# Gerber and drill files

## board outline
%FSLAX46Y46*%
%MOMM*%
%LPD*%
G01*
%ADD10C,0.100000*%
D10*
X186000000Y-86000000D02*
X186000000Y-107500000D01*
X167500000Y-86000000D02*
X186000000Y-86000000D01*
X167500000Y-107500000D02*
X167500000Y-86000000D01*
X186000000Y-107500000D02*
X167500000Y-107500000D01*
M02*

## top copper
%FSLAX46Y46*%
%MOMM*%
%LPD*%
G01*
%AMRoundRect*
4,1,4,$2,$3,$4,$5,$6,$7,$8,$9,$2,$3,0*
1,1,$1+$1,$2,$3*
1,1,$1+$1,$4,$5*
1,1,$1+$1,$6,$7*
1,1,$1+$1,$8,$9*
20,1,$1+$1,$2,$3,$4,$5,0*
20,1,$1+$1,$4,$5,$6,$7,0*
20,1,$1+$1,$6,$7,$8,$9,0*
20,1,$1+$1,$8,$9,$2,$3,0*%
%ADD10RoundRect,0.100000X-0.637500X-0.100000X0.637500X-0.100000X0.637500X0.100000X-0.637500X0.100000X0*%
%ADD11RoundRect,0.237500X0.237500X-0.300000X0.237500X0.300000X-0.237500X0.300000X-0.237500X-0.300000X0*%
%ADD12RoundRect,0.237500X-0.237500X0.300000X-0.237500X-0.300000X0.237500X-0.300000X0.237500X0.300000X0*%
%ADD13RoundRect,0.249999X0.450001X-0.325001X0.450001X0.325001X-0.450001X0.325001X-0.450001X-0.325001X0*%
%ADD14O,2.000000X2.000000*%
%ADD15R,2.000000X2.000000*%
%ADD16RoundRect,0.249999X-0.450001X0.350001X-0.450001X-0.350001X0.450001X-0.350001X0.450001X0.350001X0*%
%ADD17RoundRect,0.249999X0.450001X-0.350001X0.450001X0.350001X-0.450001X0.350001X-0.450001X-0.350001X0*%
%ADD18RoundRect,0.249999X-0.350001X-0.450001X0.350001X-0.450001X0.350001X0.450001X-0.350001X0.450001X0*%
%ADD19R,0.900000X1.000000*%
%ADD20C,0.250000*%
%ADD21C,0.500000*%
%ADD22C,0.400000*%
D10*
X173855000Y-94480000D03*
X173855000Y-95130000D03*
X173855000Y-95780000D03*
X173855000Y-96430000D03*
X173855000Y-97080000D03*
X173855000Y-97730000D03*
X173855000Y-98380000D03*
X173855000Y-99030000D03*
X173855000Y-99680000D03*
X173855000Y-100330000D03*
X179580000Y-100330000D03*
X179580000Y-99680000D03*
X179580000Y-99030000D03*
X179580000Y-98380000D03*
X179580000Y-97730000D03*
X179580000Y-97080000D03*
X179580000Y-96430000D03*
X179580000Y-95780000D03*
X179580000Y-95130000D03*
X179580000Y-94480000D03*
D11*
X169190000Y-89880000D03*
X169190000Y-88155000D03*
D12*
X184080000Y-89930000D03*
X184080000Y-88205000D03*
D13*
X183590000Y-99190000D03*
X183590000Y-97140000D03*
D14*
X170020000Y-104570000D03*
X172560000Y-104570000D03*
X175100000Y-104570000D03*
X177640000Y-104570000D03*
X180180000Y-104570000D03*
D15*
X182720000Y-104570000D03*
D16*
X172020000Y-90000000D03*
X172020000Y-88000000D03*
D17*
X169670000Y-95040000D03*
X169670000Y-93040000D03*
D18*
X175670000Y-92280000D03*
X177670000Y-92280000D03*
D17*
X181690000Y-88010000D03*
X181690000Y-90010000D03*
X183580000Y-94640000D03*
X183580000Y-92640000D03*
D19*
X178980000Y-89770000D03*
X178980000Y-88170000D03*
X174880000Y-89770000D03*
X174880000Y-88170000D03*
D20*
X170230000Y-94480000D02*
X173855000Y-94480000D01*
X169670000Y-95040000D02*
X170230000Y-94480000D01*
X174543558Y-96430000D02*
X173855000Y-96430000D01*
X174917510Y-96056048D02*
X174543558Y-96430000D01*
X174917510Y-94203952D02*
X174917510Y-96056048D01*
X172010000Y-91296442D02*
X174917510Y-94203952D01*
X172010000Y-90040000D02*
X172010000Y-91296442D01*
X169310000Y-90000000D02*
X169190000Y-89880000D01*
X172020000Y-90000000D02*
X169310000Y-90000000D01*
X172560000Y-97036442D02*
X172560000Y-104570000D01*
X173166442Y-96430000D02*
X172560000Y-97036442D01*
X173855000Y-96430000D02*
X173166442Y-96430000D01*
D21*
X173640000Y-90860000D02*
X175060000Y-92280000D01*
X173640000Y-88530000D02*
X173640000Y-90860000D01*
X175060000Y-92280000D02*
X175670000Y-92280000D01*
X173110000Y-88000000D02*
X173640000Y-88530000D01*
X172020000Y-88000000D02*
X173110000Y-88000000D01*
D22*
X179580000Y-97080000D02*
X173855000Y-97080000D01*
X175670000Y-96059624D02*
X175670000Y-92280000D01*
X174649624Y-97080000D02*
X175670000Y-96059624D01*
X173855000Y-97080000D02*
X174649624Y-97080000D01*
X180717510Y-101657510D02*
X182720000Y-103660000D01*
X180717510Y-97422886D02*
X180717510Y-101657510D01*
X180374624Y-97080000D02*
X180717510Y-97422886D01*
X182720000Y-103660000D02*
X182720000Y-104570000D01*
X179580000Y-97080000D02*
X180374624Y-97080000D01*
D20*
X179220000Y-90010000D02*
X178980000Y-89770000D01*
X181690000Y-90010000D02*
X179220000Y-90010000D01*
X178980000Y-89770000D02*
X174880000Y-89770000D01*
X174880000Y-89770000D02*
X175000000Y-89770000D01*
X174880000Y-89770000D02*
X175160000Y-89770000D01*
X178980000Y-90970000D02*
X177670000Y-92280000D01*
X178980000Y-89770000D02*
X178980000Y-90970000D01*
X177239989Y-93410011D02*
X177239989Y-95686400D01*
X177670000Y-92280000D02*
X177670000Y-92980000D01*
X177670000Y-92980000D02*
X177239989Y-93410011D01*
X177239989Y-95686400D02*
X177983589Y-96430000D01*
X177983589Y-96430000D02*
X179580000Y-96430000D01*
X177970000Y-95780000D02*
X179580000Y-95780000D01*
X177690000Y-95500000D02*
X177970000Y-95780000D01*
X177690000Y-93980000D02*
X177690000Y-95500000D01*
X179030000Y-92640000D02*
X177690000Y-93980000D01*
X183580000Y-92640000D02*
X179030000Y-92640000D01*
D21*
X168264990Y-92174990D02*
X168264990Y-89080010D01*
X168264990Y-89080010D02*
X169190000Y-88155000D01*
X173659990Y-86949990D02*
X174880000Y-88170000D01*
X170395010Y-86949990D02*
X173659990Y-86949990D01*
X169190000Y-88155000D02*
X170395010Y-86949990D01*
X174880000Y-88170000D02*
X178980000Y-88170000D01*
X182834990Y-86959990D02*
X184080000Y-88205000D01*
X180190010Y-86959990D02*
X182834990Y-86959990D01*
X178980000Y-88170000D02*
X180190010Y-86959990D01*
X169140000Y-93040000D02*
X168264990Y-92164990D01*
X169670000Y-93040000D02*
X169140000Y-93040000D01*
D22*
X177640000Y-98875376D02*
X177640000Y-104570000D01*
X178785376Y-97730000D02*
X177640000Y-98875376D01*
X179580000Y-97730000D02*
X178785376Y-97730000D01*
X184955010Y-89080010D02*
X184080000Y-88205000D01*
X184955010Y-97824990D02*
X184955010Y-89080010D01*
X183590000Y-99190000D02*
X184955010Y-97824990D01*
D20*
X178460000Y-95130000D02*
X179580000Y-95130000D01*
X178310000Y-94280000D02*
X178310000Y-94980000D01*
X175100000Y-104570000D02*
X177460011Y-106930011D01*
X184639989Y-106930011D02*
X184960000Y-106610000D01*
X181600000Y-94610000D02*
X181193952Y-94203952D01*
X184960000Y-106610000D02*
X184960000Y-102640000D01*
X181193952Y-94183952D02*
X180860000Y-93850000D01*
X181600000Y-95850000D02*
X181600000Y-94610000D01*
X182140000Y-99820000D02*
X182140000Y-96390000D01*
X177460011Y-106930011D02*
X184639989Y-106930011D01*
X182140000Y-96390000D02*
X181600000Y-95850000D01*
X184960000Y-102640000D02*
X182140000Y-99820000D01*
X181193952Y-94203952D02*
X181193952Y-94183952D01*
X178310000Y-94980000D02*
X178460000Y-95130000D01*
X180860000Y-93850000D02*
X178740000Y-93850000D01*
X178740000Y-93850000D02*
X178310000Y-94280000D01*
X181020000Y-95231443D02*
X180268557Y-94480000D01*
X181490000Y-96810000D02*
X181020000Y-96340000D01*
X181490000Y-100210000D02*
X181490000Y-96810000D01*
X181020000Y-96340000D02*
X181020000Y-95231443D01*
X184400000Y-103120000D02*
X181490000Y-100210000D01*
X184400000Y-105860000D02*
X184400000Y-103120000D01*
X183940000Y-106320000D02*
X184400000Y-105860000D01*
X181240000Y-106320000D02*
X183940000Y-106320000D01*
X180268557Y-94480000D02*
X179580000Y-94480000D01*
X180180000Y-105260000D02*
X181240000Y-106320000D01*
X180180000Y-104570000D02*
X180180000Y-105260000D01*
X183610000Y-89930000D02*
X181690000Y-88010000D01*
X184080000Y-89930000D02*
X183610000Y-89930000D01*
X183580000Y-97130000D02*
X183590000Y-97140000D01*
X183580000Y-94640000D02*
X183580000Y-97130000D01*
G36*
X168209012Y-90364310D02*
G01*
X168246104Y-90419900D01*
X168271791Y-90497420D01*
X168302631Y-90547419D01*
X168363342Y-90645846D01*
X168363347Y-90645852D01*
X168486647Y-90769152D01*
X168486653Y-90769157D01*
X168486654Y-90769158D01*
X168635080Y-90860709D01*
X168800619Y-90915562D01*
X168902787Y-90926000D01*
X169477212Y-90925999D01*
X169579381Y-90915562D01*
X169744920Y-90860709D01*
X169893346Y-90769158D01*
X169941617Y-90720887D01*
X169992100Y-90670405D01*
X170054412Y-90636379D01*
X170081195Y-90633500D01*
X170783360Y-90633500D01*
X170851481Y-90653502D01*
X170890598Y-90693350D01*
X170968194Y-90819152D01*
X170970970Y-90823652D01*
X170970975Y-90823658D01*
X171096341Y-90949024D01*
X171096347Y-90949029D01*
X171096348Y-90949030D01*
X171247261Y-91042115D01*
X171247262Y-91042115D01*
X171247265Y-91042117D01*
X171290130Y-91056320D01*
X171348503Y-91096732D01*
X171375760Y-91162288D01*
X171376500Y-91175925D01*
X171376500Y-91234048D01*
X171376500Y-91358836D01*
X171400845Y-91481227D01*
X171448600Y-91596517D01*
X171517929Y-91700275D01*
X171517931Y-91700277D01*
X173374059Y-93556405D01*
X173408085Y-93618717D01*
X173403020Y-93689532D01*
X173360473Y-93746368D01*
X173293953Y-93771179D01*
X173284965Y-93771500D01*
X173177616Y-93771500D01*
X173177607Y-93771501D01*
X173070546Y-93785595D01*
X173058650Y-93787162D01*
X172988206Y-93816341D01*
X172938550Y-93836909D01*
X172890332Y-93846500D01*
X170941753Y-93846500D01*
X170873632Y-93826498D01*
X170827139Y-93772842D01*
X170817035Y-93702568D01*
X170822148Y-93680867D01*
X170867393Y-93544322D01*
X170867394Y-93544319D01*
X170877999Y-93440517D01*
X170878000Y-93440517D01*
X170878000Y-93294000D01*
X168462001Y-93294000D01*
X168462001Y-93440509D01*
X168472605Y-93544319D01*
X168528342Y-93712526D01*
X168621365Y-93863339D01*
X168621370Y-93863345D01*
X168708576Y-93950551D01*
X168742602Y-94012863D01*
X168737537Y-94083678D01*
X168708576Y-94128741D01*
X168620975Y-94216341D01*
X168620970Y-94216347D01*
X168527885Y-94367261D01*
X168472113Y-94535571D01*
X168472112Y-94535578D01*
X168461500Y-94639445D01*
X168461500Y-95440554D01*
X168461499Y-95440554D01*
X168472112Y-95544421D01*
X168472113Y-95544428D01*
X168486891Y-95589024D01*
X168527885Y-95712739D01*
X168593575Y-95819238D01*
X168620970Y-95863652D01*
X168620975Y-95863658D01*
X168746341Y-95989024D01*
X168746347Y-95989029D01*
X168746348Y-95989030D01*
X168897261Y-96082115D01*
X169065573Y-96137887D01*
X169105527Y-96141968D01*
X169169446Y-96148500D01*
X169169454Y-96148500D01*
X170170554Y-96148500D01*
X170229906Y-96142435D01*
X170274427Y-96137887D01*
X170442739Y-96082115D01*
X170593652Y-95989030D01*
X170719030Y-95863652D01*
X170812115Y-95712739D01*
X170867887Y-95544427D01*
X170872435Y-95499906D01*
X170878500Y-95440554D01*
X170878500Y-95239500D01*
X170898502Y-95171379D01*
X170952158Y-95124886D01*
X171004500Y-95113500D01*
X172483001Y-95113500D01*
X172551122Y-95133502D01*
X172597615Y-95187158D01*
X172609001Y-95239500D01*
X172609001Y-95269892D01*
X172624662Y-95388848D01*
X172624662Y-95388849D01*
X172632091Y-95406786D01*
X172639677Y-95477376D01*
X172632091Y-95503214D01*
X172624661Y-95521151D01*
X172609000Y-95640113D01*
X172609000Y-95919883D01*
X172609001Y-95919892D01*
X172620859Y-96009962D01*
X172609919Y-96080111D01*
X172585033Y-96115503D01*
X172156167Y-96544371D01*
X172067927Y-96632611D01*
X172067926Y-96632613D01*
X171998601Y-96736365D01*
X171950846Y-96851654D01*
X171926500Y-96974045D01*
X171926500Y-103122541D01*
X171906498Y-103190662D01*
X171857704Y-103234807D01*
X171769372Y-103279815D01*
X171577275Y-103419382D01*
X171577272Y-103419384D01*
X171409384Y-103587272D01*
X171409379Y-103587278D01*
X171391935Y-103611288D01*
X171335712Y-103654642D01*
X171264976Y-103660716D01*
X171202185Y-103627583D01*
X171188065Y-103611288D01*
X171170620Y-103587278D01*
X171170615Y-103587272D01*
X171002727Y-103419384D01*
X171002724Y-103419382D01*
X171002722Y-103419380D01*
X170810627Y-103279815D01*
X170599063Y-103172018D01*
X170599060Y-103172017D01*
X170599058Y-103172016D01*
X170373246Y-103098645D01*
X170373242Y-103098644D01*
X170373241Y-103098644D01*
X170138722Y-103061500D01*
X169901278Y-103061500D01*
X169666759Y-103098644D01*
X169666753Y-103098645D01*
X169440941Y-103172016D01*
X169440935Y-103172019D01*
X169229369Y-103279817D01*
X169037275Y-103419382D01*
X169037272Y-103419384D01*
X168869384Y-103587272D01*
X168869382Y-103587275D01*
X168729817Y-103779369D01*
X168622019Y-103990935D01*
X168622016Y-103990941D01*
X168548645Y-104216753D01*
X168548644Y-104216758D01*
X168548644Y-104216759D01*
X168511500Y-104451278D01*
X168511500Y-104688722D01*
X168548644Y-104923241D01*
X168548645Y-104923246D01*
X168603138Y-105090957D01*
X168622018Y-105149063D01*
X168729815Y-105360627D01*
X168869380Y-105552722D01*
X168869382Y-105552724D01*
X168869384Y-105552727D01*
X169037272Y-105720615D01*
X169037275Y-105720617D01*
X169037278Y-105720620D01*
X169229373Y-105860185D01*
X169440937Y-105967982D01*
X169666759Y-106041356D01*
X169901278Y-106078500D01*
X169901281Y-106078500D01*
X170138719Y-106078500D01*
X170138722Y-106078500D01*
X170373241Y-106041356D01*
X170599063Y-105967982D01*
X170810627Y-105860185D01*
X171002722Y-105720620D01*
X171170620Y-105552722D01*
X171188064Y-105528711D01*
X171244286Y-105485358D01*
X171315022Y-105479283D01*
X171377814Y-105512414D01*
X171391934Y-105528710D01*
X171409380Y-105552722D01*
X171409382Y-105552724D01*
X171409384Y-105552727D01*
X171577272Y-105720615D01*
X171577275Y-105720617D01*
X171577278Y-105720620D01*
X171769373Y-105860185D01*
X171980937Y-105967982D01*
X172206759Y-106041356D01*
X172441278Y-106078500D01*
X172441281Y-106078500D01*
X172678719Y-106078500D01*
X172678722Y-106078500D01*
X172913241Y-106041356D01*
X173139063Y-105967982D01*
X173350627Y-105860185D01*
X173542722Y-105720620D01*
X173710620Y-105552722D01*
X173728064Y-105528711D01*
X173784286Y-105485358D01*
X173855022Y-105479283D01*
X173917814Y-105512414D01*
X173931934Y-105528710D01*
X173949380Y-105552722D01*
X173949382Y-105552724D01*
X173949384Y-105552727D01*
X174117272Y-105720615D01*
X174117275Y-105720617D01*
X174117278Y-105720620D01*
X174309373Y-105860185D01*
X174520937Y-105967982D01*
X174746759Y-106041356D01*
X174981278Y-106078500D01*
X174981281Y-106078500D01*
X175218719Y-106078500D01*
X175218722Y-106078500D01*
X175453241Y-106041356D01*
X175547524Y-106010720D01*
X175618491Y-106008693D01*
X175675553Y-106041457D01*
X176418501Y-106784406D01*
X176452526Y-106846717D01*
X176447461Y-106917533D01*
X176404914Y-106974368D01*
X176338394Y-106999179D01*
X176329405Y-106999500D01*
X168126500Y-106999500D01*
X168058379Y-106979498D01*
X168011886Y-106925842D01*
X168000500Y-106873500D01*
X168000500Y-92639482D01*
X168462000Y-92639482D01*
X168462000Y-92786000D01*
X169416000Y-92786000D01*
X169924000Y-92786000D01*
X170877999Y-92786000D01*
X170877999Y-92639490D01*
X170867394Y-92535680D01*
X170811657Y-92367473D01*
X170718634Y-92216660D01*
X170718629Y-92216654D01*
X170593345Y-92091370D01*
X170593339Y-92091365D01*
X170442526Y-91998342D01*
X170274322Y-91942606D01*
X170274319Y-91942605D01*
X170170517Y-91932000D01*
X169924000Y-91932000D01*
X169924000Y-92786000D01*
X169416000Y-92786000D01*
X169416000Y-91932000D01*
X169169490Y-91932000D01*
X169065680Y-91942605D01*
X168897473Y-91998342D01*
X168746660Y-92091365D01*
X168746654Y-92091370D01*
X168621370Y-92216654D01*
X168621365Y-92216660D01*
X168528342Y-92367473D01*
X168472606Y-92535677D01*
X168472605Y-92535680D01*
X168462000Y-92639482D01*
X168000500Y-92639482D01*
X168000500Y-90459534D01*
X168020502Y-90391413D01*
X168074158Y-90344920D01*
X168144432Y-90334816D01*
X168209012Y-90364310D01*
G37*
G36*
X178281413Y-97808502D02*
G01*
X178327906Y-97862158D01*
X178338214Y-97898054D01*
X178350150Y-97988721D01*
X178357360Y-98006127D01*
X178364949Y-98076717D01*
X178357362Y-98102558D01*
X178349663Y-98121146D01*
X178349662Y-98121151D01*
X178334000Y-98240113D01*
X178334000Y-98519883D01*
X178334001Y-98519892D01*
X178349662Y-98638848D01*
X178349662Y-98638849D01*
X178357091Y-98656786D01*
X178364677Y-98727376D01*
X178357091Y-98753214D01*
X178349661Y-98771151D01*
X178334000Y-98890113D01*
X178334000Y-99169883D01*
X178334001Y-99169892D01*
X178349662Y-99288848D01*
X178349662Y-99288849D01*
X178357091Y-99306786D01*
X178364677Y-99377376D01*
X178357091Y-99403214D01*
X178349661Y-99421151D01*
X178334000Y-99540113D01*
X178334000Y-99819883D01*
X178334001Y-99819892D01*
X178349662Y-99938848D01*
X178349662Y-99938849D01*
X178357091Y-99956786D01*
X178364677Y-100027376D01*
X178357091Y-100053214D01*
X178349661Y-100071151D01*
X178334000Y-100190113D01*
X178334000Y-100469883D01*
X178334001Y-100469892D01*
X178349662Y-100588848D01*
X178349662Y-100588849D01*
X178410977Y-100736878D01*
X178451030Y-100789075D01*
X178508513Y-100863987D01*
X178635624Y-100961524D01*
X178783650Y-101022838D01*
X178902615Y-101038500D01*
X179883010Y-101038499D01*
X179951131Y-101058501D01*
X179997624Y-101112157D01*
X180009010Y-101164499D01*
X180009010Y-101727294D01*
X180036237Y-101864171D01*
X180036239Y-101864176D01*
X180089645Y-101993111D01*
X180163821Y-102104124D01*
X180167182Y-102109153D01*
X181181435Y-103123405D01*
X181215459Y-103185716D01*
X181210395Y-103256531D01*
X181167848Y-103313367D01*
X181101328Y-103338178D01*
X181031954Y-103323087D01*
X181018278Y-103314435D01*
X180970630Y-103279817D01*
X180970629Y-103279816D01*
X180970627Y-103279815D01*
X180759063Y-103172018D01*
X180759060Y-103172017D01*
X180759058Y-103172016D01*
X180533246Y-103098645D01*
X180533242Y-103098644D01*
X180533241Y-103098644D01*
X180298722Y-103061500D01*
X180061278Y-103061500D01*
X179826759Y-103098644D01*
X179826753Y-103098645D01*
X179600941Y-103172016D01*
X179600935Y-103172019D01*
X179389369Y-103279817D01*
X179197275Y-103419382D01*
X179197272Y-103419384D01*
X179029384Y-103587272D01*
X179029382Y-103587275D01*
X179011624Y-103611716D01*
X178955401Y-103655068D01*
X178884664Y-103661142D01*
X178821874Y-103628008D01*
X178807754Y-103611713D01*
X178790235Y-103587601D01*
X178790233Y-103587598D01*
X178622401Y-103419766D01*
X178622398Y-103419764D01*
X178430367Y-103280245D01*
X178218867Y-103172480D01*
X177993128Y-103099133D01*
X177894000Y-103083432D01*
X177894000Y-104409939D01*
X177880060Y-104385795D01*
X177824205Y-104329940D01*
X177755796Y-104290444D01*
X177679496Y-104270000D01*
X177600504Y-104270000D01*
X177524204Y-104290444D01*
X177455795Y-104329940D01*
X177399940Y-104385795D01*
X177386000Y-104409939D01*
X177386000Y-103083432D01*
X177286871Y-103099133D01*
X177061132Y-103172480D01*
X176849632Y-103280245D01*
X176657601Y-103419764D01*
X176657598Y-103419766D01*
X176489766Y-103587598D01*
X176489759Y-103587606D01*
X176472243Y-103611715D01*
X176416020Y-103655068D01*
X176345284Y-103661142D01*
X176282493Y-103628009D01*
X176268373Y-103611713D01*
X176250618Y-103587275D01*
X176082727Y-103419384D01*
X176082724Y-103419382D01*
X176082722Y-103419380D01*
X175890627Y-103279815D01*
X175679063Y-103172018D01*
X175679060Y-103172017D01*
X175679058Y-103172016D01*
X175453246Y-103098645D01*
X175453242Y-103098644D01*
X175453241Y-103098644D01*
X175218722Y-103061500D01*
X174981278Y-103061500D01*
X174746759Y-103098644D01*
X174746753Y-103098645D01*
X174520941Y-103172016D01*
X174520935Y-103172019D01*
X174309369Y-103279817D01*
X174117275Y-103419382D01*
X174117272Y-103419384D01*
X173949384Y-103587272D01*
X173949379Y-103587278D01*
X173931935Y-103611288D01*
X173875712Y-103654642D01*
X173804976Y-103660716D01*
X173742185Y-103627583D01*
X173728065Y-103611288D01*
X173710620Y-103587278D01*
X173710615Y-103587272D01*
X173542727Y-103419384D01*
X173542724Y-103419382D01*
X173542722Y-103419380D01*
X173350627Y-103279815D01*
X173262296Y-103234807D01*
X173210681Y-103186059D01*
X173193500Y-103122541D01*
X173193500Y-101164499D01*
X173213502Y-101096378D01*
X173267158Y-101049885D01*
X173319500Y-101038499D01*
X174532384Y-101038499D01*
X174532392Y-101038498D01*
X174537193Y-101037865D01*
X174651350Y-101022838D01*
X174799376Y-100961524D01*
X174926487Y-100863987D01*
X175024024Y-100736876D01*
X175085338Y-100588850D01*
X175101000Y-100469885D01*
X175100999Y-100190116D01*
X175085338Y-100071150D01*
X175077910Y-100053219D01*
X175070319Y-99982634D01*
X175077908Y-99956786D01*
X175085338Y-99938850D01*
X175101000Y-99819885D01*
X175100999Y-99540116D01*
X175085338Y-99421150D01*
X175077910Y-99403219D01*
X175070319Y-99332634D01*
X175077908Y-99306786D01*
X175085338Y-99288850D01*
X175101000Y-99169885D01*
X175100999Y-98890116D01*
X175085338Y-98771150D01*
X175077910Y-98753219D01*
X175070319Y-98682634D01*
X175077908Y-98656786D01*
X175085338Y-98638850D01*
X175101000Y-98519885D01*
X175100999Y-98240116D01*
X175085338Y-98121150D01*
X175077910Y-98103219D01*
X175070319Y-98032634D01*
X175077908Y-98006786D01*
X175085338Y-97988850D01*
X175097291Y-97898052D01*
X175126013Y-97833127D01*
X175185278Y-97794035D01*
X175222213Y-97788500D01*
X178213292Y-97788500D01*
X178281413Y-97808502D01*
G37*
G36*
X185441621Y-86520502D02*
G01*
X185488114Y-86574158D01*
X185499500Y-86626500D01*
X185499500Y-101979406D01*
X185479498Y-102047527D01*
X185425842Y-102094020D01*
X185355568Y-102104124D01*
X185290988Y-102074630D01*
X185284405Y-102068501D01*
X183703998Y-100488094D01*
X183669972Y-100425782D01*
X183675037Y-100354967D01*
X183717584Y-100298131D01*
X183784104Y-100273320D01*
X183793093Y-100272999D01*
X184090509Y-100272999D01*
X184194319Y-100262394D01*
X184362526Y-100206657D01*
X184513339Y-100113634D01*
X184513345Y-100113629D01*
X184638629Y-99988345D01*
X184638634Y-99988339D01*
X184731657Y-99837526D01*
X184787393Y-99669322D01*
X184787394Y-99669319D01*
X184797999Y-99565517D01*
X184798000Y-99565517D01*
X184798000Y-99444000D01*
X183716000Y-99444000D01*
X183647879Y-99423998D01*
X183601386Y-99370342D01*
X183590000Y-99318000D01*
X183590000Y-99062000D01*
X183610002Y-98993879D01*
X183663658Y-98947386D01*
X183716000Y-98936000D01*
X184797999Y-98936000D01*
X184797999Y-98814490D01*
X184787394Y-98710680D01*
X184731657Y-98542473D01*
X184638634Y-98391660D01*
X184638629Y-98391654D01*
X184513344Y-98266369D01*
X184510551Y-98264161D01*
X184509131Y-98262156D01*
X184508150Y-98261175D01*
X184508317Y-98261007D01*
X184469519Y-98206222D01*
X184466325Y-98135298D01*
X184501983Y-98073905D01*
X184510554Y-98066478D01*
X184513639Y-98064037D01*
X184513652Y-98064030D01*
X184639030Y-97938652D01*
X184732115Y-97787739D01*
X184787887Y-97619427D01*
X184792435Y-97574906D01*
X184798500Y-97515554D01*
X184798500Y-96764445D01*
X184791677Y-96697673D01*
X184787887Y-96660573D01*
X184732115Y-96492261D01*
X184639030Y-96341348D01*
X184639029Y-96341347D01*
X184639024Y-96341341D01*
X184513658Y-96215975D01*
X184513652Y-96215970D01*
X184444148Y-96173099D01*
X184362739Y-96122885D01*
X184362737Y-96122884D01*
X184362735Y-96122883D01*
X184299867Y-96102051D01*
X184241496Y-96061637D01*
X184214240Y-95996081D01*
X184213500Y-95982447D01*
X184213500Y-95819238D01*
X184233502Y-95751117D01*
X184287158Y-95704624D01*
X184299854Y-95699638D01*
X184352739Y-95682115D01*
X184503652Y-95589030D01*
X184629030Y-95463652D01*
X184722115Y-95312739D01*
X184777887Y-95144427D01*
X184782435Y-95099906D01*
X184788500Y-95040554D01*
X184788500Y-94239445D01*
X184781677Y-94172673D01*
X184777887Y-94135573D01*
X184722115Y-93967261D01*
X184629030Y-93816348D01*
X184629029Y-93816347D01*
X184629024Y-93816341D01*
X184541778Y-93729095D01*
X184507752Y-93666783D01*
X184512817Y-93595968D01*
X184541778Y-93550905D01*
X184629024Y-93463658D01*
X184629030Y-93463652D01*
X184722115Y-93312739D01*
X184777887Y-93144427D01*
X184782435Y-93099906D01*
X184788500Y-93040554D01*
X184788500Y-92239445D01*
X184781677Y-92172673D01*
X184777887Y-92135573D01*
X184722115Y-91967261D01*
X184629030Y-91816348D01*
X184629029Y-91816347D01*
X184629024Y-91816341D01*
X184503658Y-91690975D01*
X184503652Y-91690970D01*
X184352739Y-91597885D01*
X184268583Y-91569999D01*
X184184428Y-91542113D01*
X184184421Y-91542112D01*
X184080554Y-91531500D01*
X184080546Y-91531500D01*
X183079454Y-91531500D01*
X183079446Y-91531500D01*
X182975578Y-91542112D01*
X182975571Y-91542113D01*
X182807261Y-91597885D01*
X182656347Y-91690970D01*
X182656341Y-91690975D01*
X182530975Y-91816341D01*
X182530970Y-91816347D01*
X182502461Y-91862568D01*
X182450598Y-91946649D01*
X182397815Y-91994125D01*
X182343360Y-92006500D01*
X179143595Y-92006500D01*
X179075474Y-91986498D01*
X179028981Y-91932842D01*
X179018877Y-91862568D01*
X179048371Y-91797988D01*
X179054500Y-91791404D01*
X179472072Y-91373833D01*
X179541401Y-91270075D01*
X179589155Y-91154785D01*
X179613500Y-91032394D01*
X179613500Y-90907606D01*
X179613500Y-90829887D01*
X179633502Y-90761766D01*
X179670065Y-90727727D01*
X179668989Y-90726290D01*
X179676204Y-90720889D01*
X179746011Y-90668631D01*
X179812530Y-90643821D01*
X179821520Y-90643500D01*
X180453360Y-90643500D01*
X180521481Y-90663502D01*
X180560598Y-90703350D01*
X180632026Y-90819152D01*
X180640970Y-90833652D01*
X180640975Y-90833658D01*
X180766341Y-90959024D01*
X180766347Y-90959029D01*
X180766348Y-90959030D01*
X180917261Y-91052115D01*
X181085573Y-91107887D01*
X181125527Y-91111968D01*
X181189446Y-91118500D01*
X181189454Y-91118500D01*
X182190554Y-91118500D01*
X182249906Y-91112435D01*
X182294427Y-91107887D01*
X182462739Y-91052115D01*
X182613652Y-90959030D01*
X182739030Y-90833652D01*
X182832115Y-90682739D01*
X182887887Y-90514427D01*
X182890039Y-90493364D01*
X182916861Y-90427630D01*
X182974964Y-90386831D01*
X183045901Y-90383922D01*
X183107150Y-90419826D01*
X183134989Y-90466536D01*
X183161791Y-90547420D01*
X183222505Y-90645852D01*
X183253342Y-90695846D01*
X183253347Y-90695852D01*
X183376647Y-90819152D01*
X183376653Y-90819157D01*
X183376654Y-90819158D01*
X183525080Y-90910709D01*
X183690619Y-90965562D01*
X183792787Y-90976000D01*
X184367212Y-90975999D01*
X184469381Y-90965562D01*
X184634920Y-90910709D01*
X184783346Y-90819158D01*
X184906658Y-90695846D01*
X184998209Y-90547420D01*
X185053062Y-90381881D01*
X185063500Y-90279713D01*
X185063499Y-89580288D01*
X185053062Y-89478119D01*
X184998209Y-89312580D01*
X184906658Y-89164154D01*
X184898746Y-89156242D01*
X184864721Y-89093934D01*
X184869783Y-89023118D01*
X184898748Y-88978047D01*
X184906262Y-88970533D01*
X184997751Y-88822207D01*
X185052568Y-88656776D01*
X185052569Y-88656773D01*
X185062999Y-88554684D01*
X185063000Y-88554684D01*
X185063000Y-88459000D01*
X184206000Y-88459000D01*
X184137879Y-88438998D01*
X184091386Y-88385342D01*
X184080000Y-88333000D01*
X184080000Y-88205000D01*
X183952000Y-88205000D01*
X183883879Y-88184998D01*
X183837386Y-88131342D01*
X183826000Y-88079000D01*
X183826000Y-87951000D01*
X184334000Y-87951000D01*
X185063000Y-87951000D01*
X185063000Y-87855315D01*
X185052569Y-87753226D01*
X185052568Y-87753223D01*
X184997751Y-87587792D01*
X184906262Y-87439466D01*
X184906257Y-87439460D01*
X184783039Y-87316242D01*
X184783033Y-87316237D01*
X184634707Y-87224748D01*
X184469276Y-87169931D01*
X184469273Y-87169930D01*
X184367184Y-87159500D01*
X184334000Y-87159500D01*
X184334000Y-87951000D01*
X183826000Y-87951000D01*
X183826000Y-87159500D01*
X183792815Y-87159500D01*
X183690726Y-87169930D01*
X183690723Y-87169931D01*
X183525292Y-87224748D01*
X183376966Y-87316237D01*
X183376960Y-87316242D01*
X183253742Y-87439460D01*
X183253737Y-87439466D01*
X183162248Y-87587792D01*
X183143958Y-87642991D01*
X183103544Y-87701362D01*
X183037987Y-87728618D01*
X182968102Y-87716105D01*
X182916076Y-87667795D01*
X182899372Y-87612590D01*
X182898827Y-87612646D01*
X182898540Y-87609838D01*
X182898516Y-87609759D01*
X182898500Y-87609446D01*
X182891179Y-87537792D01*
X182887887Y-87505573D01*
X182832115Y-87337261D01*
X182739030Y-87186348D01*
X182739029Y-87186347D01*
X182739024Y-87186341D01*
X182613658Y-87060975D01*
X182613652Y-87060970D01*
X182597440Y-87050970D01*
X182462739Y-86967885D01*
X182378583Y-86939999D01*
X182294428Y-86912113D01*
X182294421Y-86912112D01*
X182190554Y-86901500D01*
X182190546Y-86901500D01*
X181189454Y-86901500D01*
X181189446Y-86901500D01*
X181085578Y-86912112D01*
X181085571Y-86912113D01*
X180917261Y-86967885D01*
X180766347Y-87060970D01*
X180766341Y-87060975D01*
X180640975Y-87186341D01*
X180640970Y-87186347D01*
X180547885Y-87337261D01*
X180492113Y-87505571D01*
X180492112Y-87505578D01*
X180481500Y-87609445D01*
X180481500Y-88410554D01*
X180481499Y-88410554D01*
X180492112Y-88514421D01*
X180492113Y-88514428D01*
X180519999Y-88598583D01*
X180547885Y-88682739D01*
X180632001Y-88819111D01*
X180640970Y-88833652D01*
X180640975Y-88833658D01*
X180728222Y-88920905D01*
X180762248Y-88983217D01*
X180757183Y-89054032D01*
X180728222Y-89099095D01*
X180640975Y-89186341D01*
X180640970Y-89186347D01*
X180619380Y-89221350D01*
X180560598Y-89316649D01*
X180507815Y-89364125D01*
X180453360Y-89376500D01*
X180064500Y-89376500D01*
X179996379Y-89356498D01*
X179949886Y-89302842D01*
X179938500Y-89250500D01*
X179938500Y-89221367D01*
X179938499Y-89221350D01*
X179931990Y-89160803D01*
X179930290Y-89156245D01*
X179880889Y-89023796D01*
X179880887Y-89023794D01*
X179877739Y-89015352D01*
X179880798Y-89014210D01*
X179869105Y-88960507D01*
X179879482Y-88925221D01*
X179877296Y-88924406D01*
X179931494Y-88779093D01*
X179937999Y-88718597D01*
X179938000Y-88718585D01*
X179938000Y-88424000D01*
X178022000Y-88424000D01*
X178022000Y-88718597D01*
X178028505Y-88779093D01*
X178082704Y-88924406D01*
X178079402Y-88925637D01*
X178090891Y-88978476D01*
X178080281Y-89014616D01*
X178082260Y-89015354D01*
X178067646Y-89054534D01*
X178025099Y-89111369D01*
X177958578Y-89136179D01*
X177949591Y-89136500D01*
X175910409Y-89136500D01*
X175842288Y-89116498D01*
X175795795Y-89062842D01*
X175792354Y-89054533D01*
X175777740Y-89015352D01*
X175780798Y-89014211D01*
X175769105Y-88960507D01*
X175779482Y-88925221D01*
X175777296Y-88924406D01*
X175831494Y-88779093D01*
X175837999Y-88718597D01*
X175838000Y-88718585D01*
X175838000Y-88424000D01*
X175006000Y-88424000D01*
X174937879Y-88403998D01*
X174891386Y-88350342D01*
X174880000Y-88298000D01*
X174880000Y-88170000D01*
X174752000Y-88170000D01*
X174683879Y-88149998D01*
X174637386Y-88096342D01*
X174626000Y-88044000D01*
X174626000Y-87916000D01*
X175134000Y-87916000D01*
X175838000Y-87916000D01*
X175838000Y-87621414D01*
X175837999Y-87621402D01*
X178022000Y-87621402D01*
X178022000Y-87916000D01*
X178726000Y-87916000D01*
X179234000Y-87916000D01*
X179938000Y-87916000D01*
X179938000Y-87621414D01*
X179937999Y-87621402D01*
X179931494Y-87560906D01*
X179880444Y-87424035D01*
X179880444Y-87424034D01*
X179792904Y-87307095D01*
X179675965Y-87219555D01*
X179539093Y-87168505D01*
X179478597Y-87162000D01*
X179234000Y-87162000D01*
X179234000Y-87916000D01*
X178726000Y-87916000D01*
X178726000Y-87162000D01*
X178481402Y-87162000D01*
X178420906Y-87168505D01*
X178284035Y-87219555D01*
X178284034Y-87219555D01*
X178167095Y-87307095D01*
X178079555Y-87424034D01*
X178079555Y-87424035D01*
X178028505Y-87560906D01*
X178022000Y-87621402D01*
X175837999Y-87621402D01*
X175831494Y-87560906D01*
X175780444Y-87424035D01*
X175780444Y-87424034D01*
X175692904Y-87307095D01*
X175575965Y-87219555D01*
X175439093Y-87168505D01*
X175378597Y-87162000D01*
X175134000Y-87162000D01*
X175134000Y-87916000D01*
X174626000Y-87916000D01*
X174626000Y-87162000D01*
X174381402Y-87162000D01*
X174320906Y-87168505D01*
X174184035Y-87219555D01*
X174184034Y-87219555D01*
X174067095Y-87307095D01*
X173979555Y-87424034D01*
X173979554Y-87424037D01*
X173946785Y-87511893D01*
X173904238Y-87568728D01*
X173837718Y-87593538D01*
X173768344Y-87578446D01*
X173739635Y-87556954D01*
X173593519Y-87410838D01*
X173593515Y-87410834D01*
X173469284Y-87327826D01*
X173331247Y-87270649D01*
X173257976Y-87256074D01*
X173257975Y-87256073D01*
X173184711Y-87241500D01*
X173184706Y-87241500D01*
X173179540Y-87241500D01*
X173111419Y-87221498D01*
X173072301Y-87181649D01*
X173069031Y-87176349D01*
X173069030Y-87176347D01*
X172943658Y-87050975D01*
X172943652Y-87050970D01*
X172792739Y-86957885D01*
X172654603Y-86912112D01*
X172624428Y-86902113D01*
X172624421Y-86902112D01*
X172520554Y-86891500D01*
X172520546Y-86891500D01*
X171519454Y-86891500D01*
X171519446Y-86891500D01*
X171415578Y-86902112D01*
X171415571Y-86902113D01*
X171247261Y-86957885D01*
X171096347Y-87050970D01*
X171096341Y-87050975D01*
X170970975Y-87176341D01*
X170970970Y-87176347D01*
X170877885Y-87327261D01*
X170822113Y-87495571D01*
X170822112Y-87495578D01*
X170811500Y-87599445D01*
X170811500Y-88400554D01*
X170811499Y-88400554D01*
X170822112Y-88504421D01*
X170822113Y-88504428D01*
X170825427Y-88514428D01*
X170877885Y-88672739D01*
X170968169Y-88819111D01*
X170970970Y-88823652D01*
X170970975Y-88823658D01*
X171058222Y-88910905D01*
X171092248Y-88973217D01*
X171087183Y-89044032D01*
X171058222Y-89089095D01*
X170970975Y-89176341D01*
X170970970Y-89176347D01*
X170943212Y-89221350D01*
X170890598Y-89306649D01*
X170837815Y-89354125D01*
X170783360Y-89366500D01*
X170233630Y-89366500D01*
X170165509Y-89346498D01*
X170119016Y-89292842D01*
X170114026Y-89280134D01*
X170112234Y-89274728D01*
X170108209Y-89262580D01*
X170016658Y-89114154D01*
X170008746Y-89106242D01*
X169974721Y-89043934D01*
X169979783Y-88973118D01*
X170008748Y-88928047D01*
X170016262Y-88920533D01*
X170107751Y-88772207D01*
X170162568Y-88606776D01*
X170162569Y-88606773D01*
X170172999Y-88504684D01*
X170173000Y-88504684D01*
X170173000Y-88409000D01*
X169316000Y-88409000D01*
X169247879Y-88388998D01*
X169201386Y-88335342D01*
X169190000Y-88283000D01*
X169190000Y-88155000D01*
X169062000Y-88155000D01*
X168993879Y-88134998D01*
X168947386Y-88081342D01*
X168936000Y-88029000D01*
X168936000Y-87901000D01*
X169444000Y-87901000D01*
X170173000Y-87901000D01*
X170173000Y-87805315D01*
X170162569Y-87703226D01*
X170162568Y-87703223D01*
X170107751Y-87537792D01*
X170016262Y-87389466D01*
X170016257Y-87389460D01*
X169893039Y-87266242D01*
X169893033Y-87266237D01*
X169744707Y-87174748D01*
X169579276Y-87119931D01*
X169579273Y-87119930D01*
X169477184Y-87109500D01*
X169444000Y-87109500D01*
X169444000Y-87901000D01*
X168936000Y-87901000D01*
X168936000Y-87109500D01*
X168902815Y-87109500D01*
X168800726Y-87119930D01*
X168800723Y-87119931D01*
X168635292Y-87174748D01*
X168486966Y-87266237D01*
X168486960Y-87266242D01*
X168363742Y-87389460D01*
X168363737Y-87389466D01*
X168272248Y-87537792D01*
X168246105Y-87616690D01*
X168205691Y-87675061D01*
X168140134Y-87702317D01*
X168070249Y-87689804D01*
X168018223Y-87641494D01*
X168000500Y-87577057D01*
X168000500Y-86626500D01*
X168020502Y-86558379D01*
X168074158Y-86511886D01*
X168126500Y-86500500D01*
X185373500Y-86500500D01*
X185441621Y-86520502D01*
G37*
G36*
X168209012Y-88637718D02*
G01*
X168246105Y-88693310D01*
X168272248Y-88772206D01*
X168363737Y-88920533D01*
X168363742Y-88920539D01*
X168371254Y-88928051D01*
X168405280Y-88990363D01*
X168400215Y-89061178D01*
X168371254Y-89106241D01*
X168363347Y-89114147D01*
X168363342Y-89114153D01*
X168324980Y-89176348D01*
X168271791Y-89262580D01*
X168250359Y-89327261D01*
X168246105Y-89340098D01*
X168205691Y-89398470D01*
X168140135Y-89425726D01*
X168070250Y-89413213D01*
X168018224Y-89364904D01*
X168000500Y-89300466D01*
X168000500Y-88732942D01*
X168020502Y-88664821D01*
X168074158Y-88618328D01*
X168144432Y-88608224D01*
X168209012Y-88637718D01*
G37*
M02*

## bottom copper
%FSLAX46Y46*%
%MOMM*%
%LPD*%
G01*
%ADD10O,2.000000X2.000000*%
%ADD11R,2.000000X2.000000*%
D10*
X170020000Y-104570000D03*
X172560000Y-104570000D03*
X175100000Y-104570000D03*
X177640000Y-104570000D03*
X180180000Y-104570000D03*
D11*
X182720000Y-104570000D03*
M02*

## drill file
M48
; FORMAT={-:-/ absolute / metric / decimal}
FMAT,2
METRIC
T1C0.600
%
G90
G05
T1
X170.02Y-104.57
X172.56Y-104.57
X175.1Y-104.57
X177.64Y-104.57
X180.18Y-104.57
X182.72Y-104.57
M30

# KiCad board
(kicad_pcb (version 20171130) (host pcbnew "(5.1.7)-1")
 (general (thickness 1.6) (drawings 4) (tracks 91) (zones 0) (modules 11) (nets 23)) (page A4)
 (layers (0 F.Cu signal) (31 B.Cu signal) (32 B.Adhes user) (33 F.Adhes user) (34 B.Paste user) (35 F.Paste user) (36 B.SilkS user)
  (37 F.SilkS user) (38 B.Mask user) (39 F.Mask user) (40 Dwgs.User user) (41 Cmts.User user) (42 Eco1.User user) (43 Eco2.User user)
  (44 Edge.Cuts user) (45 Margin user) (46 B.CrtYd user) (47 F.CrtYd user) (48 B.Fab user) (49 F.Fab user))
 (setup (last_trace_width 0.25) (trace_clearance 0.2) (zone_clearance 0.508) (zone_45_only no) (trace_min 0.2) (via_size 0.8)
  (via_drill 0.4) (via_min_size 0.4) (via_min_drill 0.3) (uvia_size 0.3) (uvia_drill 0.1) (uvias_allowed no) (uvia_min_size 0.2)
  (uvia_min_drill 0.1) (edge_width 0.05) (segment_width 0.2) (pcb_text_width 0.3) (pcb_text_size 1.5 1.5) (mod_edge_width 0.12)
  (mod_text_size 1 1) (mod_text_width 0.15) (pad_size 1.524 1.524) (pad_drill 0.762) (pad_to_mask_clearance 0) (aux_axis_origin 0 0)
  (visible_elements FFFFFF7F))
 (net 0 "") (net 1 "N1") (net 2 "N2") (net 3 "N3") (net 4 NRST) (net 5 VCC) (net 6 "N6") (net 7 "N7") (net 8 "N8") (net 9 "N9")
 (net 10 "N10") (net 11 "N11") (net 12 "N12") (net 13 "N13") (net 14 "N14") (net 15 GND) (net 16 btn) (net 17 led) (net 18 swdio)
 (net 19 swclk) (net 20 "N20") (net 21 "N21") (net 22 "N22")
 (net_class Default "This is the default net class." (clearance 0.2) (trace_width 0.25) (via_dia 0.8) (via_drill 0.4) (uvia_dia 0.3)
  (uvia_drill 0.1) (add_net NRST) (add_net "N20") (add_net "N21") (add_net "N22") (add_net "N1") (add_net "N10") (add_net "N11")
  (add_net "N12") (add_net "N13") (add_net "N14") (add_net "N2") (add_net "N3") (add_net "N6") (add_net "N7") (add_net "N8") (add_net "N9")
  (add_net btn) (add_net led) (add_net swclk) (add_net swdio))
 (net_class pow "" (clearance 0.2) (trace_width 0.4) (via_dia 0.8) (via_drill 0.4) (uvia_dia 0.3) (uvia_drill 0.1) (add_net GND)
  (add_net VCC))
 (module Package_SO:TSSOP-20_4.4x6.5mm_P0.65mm (layer F.Cu) (at 176.7175 97.405)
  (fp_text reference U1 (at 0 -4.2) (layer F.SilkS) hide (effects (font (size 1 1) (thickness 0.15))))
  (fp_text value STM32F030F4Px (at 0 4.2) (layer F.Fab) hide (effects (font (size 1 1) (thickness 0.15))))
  (pad 1 smd roundrect (at -2.8625 -2.925) (size 1.475 0.4) (layers F.Cu F.Paste F.Mask) (roundrect_rratio 0.25) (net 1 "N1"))
  (pad 2 smd roundrect (at -2.8625 -2.275) (size 1.475 0.4) (layers F.Cu F.Paste F.Mask) (roundrect_rratio 0.25) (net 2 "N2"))
  (pad 3 smd roundrect (at -2.8625 -1.625) (size 1.475 0.4) (layers F.Cu F.Paste F.Mask) (roundrect_rratio 0.25) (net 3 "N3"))
  (pad 4 smd roundrect (at -2.8625 -0.975) (size 1.475 0.4) (layers F.Cu F.Paste F.Mask) (roundrect_rratio 0.25) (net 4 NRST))
  (pad 5 smd roundrect (at -2.8625 -0.325) (size 1.475 0.4) (layers F.Cu F.Paste F.Mask) (roundrect_rratio 0.25) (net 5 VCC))
  (pad 6 smd roundrect (at -2.8625 0.325) (size 1.475 0.4) (layers F.Cu F.Paste F.Mask) (roundrect_rratio 0.25) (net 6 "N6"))
  (pad 7 smd roundrect (at -2.8625 0.975) (size 1.475 0.4) (layers F.Cu F.Paste F.Mask) (roundrect_rratio 0.25) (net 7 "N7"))
  (pad 8 smd roundrect (at -2.8625 1.625) (size 1.475 0.4) (layers F.Cu F.Paste F.Mask) (roundrect_rratio 0.25) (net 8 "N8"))
  (pad 9 smd roundrect (at -2.8625 2.275) (size 1.475 0.4) (layers F.Cu F.Paste F.Mask) (roundrect_rratio 0.25) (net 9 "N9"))
  (pad 10 smd roundrect (at -2.8625 2.925) (size 1.475 0.4) (layers F.Cu F.Paste F.Mask) (roundrect_rratio 0.25) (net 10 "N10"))
  (pad 11 smd roundrect (at 2.8625 2.925) (size 1.475 0.4) (layers F.Cu F.Paste F.Mask) (roundrect_rratio 0.25) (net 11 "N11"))
  (pad 12 smd roundrect (at 2.8625 2.275) (size 1.475 0.4) (layers F.Cu F.Paste F.Mask) (roundrect_rratio 0.25) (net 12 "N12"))
  (pad 13 smd roundrect (at 2.8625 1.625) (size 1.475 0.4) (layers F.Cu F.Paste F.Mask) (roundrect_rratio 0.25) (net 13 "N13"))
  (pad 14 smd roundrect (at 2.8625 0.975) (size 1.475 0.4) (layers F.Cu F.Paste F.Mask) (roundrect_rratio 0.25) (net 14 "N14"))
  (pad 15 smd roundrect (at 2.8625 0.325) (size 1.475 0.4) (layers F.Cu F.Paste F.Mask) (roundrect_rratio 0.25) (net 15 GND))
  (pad 16 smd roundrect (at 2.8625 -0.325) (size 1.475 0.4) (layers F.Cu F.Paste F.Mask) (roundrect_rratio 0.25) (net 5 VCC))
  (pad 17 smd roundrect (at 2.8625 -0.975) (size 1.475 0.4) (layers F.Cu F.Paste F.Mask) (roundrect_rratio 0.25) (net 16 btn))
  (pad 18 smd roundrect (at 2.8625 -1.625) (size 1.475 0.4) (layers F.Cu F.Paste F.Mask) (roundrect_rratio 0.25) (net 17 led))
  (pad 19 smd roundrect (at 2.8625 -2.275) (size 1.475 0.4) (layers F.Cu F.Paste F.Mask) (roundrect_rratio 0.25) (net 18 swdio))
  (pad 20 smd roundrect (at 2.8625 -2.925) (size 1.475 0.4) (layers F.Cu F.Paste F.Mask) (roundrect_rratio 0.25) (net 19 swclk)))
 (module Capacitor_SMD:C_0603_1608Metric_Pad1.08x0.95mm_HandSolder (layer F.Cu) (at 169.19 89.0175 90)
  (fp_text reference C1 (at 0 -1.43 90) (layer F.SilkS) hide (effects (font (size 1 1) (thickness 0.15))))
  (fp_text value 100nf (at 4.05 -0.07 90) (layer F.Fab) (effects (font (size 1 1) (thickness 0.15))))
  (pad 1 smd roundrect (at -0.8625 0 90) (size 1.075 0.95) (layers F.Cu F.Paste F.Mask) (roundrect_rratio 0.25) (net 4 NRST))
  (pad 2 smd roundrect (at 0.8625 0 90) (size 1.075 0.95) (layers F.Cu F.Paste F.Mask) (roundrect_rratio 0.25) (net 15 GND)))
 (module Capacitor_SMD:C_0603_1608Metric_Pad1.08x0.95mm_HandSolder (layer F.Cu) (at 184.08 89.0675 270)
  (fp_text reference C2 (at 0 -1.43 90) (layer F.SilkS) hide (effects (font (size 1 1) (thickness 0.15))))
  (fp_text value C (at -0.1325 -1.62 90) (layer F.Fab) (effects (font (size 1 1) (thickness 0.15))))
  (pad 2 smd roundrect (at 0.8625 0 270) (size 1.075 0.95) (layers F.Cu F.Paste F.Mask) (roundrect_rratio 0.25) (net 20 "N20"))
  (pad 1 smd roundrect (at -0.8625 0 270) (size 1.075 0.95) (layers F.Cu F.Paste F.Mask) (roundrect_rratio 0.25) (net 15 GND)))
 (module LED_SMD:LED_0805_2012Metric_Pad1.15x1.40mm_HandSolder (layer F.Cu) (at 183.59 98.165 90)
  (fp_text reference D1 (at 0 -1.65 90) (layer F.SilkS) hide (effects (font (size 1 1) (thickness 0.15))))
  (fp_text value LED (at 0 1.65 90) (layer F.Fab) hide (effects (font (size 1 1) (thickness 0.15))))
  (pad 1 smd roundrect (at -1.025 0 90) (size 1.15 1.4) (layers F.Cu F.Paste F.Mask) (roundrect_rratio 0.2173904347826087) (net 15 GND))
  (pad 2 smd roundrect (at 1.025 0 90) (size 1.15 1.4) (layers F.Cu F.Paste F.Mask) (roundrect_rratio 0.2173904347826087) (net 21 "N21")))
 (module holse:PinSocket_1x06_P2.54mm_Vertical (layer F.Cu) (at 182.72 104.57 270)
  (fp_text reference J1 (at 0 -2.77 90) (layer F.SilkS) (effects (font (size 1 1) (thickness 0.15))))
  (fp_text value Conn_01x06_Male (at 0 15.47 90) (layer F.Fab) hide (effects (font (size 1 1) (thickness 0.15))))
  (pad 6 thru_hole oval (at 0 12.7 270) (size 2 2) (drill 0.6) (layers *.Cu *.Mask) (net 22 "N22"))
  (pad 5 thru_hole oval (at 0 10.16 270) (size 2 2) (drill 0.6) (layers *.Cu *.Mask) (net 4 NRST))
  (pad 4 thru_hole oval (at 0 7.62 270) (size 2 2) (drill 0.6) (layers *.Cu *.Mask) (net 18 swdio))
  (pad 3 thru_hole oval (at 0 5.08 270) (size 2 2) (drill 0.6) (layers *.Cu *.Mask) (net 15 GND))
  (pad 2 thru_hole oval (at 0 2.54 270) (size 2 2) (drill 0.6) (layers *.Cu *.Mask) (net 19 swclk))
  (pad 1 thru_hole rect (at 0 0 270) (size 2 2) (drill 0.6) (layers *.Cu *.Mask) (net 5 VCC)))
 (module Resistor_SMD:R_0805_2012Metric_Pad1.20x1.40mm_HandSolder (layer F.Cu) (at 172.02 89 270)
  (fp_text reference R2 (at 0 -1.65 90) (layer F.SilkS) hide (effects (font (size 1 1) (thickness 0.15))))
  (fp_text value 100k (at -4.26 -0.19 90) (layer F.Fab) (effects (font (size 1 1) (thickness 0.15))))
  (pad 2 smd roundrect (at 1 0 270) (size 1.2 1.4) (layers F.Cu F.Paste F.Mask) (roundrect_rratio 0.2083325) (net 4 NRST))
  (pad 1 smd roundrect (at -1 0 270) (size 1.2 1.4) (layers F.Cu F.Paste F.Mask) (roundrect_rratio 0.2083325) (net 5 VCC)))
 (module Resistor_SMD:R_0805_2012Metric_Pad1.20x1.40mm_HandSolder (layer F.Cu) (at 169.67 94.04 90)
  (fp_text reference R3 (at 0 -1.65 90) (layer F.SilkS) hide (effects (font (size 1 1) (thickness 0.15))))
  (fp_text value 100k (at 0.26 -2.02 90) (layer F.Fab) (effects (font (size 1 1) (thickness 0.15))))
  (pad 1 smd roundrect (at -1 0 90) (size 1.2 1.4) (layers F.Cu F.Paste F.Mask) (roundrect_rratio 0.2083325) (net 1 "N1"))
  (pad 2 smd roundrect (at 1 0 90) (size 1.2 1.4) (layers F.Cu F.Paste F.Mask) (roundrect_rratio 0.2083325) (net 15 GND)))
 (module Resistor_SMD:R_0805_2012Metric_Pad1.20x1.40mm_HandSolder (layer F.Cu) (at 176.67 92.28)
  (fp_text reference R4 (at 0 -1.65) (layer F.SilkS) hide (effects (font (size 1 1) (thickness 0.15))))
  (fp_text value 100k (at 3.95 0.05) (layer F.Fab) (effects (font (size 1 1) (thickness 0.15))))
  (pad 1 smd roundrect (at -1 0) (size 1.2 1.4) (layers F.Cu F.Paste F.Mask) (roundrect_rratio 0.2083325) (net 5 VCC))
  (pad 2 smd roundrect (at 1 0) (size 1.2 1.4) (layers F.Cu F.Paste F.Mask) (roundrect_rratio 0.2083325) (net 16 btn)))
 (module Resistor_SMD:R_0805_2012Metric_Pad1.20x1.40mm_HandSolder (layer F.Cu) (at 181.69 89.01 90)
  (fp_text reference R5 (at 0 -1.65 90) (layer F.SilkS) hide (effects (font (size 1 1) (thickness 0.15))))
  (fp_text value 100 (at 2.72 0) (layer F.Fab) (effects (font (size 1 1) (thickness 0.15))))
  (pad 2 smd roundrect (at 1 0 90) (size 1.2 1.4) (layers F.Cu F.Paste F.Mask) (roundrect_rratio 0.2083325) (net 20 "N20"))
  (pad 1 smd roundrect (at -1 0 90) (size 1.2 1.4) (layers F.Cu F.Paste F.Mask) (roundrect_rratio 0.2083325) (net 16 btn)))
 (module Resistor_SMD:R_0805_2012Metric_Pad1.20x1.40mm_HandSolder (layer F.Cu) (at 183.58 93.64 90)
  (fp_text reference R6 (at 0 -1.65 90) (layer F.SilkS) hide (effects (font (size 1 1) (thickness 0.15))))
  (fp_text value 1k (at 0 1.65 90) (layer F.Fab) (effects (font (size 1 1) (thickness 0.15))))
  (pad 1 smd roundrect (at -1 0 90) (size 1.2 1.4) (layers F.Cu F.Paste F.Mask) (roundrect_rratio 0.2083325) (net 21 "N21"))
  (pad 2 smd roundrect (at 1 0 90) (size 1.2 1.4) (layers F.Cu F.Paste F.Mask) (roundrect_rratio 0.2083325) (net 17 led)))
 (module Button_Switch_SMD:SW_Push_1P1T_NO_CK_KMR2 (layer F.Cu) (at 176.93 88.97 180)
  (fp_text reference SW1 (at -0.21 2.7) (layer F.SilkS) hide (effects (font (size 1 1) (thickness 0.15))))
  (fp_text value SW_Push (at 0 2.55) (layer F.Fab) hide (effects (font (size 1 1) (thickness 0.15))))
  (pad 1 smd rect (at -2.05 -0.8 180) (size 0.9 1) (layers F.Cu F.Paste F.Mask) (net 16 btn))
  (pad 2 smd rect (at -2.05 0.8 180) (size 0.9 1) (layers F.Cu F.Paste F.Mask) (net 15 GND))
  (pad 1 smd rect (at 2.05 -0.8 180) (size 0.9 1) (layers F.Cu F.Paste F.Mask) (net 16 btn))
  (pad 2 smd rect (at 2.05 0.8 180) (size 0.9 1) (layers F.Cu F.Paste F.Mask) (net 15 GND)))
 (gr_line (start 186 86) (end 186 107.5) (layer Edge.Cuts) (width 0.1))
 (gr_line (start 167.5 86) (end 186 86) (layer Edge.Cuts) (width 0.1))
 (gr_line (start 167.5 107.5) (end 167.5 86) (layer Edge.Cuts) (width 0.1))
 (gr_line (start 186 107.5) (end 167.5 107.5) (layer Edge.Cuts) (width 0.1))
 (segment (start 170.23 94.48) (end 173.855 94.48) (width 0.25) (layer F.Cu) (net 1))
 (segment (start 169.67 95.04) (end 170.23 94.48) (width 0.25) (layer F.Cu) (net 1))
 (segment (start 174.543558 96.43) (end 173.855 96.43) (width 0.25) (layer F.Cu) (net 4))
 (segment (start 174.91751 96.056048) (end 174.543558 96.43) (width 0.25) (layer F.Cu) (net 4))
 (segment (start 174.91751 94.203952) (end 174.91751 96.056048) (width 0.25) (layer F.Cu) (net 4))
 (segment (start 172.01 91.296442) (end 174.91751 94.203952) (width 0.25) (layer F.Cu) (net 4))
 (segment (start 172.01 90.04) (end 172.01 91.296442) (width 0.25) (layer F.Cu) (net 4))
 (segment (start 169.31 90) (end 169.19 89.88) (width 0.25) (layer F.Cu) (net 4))
 (segment (start 172.02 90) (end 169.31 90) (width 0.25) (layer F.Cu) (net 4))
 (segment (start 172.56 97.036442) (end 172.56 104.57) (width 0.25) (layer F.Cu) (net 4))
 (segment (start 173.166442 96.43) (end 172.56 97.036442) (width 0.25) (layer F.Cu) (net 4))
 (segment (start 173.855 96.43) (end 173.166442 96.43) (width 0.25) (layer F.Cu) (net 4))
 (segment (start 173.64 90.86) (end 175.06 92.28) (width 0.5) (layer F.Cu) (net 5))
 (segment (start 173.64 88.53) (end 173.64 90.86) (width 0.5) (layer F.Cu) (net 5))
 (segment (start 175.06 92.28) (end 175.67 92.28) (width 0.5) (layer F.Cu) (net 5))
 (segment (start 173.11 88) (end 173.64 88.53) (width 0.5) (layer F.Cu) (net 5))
 (segment (start 172.02 88) (end 173.11 88) (width 0.5) (layer F.Cu) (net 5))
 (segment (start 179.58 97.08) (end 173.855 97.08) (width 0.4) (layer F.Cu) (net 5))
 (segment (start 175.67 96.059624) (end 175.67 92.28) (width 0.4) (layer F.Cu) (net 5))
 (segment (start 174.649624 97.08) (end 175.67 96.059624) (width 0.4) (layer F.Cu) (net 5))
 (segment (start 173.855 97.08) (end 174.649624 97.08) (width 0.4) (layer F.Cu) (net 5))
 (segment (start 180.71751 101.65751) (end 182.72 103.66) (width 0.4) (layer F.Cu) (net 5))
 (segment (start 180.71751 97.422886) (end 180.71751 101.65751) (width 0.4) (layer F.Cu) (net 5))
 (segment (start 180.374624 97.08) (end 180.71751 97.422886) (width 0.4) (layer F.Cu) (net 5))
 (segment (start 182.72 103.66) (end 182.72 104.57) (width 0.4) (layer F.Cu) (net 5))
 (segment (start 179.58 97.08) (end 180.374624 97.08) (width 0.4) (layer F.Cu) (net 5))
 (segment (start 179.22 90.01) (end 178.98 89.77) (width 0.25) (layer F.Cu) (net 16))
 (segment (start 181.69 90.01) (end 179.22 90.01) (width 0.25) (layer F.Cu) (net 16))
 (segment (start 178.98 89.77) (end 174.88 89.77) (width 0.25) (layer F.Cu) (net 16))
 (segment (start 174.88 89.77) (end 175 89.77) (width 0.25) (layer F.Cu) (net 16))
 (segment (start 174.88 89.77) (end 175.16 89.77) (width 0.25) (layer F.Cu) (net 16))
 (segment (start 178.98 90.97) (end 177.67 92.28) (width 0.25) (layer F.Cu) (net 16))
 (segment (start 178.98 89.77) (end 178.98 90.97) (width 0.25) (layer F.Cu) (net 16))
 (segment (start 177.239989 93.410011) (end 177.239989 95.6864) (width 0.25) (layer F.Cu) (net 16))
 (segment (start 177.67 92.28) (end 177.67 92.98) (width 0.25) (layer F.Cu) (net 16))
 (segment (start 177.67 92.98) (end 177.239989 93.410011) (width 0.25) (layer F.Cu) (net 16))
 (segment (start 177.239989 95.6864) (end 177.983589 96.43) (width 0.25) (layer F.Cu) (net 16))
 (segment (start 177.983589 96.43) (end 179.58 96.43) (width 0.25) (layer F.Cu) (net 16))
 (segment (start 177.97 95.78) (end 179.58 95.78) (width 0.25) (layer F.Cu) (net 17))
 (segment (start 177.69 95.5) (end 177.97 95.78) (width 0.25) (layer F.Cu) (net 17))
 (segment (start 177.69 93.98) (end 177.69 95.5) (width 0.25) (layer F.Cu) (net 17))
 (segment (start 179.03 92.64) (end 177.69 93.98) (width 0.25) (layer F.Cu) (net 17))
 (segment (start 183.58 92.64) (end 179.03 92.64) (width 0.25) (layer F.Cu) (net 17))
 (segment (start 168.26499 92.17499) (end 168.26499 89.08001) (width 0.5) (layer F.Cu) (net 15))
 (segment (start 168.26499 89.08001) (end 169.19 88.155) (width 0.5) (layer F.Cu) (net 15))
 (segment (start 173.65999 86.94999) (end 174.88 88.17) (width 0.5) (layer F.Cu) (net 15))
 (segment (start 170.39501 86.94999) (end 173.65999 86.94999) (width 0.5) (layer F.Cu) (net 15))
 (segment (start 169.19 88.155) (end 170.39501 86.94999) (width 0.5) (layer F.Cu) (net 15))
 (segment (start 174.88 88.17) (end 178.98 88.17) (width 0.5) (layer F.Cu) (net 15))
 (segment (start 182.83499 86.95999) (end 184.08 88.205) (width 0.5) (layer F.Cu) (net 15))
 (segment (start 180.19001 86.95999) (end 182.83499 86.95999) (width 0.5) (layer F.Cu) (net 15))
 (segment (start 178.98 88.17) (end 180.19001 86.95999) (width 0.5) (layer F.Cu) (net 15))
 (segment (start 169.14 93.04) (end 168.26499 92.16499) (width 0.5) (layer F.Cu) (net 15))
 (segment (start 169.67 93.04) (end 169.14 93.04) (width 0.5) (layer F.Cu) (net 15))
 (segment (start 177.64 98.875376) (end 177.64 104.57) (width 0.4) (layer F.Cu) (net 15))
 (segment (start 178.785376 97.73) (end 177.64 98.875376) (width 0.4) (layer F.Cu) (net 15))
 (segment (start 179.58 97.73) (end 178.785376 97.73) (width 0.4) (layer F.Cu) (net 15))
 (segment (start 184.95501 89.08001) (end 184.08 88.205) (width 0.4) (layer F.Cu) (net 15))
 (segment (start 184.95501 97.82499) (end 184.95501 89.08001) (width 0.4) (layer F.Cu) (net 15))
 (segment (start 183.59 99.19) (end 184.95501 97.82499) (width 0.4) (layer F.Cu) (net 15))
 (segment (start 178.46 95.13) (end 179.58 95.13) (width 0.25) (layer F.Cu) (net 18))
 (segment (start 178.31 94.28) (end 178.31 94.98) (width 0.25) (layer F.Cu) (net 18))
 (segment (start 175.1 104.57) (end 177.460011 106.930011) (width 0.25) (layer F.Cu) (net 18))
 (segment (start 184.639989 106.930011) (end 184.96 106.61) (width 0.25) (layer F.Cu) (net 18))
 (segment (start 181.6 94.61) (end 181.193952 94.203952) (width 0.25) (layer F.Cu) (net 18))
 (segment (start 184.96 106.61) (end 184.96 102.64) (width 0.25) (layer F.Cu) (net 18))
 (segment (start 181.193952 94.183952) (end 180.86 93.85) (width 0.25) (layer F.Cu) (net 18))
 (segment (start 181.6 95.85) (end 181.6 94.61) (width 0.25) (layer F.Cu) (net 18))
 (segment (start 182.14 99.82) (end 182.14 96.39) (width 0.25) (layer F.Cu) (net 18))
 (segment (start 177.460011 106.930011) (end 184.639989 106.930011) (width 0.25) (layer F.Cu) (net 18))
 (segment (start 182.14 96.39) (end 181.6 95.85) (width 0.25) (layer F.Cu) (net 18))
 (segment (start 184.96 102.64) (end 182.14 99.82) (width 0.25) (layer F.Cu) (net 18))
 (segment (start 181.193952 94.203952) (end 181.193952 94.183952) (width 0.25) (layer F.Cu) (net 18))
 (segment (start 178.31 94.98) (end 178.46 95.13) (width 0.25) (layer F.Cu) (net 18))
 (segment (start 180.86 93.85) (end 178.74 93.85) (width 0.25) (layer F.Cu) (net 18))
 (segment (start 178.74 93.85) (end 178.31 94.28) (width 0.25) (layer F.Cu) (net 18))
 (segment (start 181.02 95.231443) (end 180.268557 94.48) (width 0.25) (layer F.Cu) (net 19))
 (segment (start 181.49 96.81) (end 181.02 96.34) (width 0.25) (layer F.Cu) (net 19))
 (segment (start 181.49 100.21) (end 181.49 96.81) (width 0.25) (layer F.Cu) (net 19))
 (segment (start 181.02 96.34) (end 181.02 95.231443) (width 0.25) (layer F.Cu) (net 19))
 (segment (start 184.4 103.12) (end 181.49 100.21) (width 0.25) (layer F.Cu) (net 19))
 (segment (start 184.4 105.86) (end 184.4 103.12) (width 0.25) (layer F.Cu) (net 19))
 (segment (start 183.94 106.32) (end 184.4 105.86) (width 0.25) (layer F.Cu) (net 19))
 (segment (start 181.24 106.32) (end 183.94 106.32) (width 0.25) (layer F.Cu) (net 19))
 (segment (start 180.268557 94.48) (end 179.58 94.48) (width 0.25) (layer F.Cu) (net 19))
 (segment (start 180.18 105.26) (end 181.24 106.32) (width 0.25) (layer F.Cu) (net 19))
 (segment (start 180.18 104.57) (end 180.18 105.26) (width 0.25) (layer F.Cu) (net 19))
 (segment (start 183.61 89.93) (end 181.69 88.01) (width 0.25) (layer F.Cu) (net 20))
 (segment (start 184.08 89.93) (end 183.61 89.93) (width 0.25) (layer F.Cu) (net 20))
 (segment (start 183.58 97.13) (end 183.59 97.14) (width 0.25) (layer F.Cu) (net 21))
 (segment (start 183.58 94.64) (end 183.58 97.13) (width 0.25) (layer F.Cu) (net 21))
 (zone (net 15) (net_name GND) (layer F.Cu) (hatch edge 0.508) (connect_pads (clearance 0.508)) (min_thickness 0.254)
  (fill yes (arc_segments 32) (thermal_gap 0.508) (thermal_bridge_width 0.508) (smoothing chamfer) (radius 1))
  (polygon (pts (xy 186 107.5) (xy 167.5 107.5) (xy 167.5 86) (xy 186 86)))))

